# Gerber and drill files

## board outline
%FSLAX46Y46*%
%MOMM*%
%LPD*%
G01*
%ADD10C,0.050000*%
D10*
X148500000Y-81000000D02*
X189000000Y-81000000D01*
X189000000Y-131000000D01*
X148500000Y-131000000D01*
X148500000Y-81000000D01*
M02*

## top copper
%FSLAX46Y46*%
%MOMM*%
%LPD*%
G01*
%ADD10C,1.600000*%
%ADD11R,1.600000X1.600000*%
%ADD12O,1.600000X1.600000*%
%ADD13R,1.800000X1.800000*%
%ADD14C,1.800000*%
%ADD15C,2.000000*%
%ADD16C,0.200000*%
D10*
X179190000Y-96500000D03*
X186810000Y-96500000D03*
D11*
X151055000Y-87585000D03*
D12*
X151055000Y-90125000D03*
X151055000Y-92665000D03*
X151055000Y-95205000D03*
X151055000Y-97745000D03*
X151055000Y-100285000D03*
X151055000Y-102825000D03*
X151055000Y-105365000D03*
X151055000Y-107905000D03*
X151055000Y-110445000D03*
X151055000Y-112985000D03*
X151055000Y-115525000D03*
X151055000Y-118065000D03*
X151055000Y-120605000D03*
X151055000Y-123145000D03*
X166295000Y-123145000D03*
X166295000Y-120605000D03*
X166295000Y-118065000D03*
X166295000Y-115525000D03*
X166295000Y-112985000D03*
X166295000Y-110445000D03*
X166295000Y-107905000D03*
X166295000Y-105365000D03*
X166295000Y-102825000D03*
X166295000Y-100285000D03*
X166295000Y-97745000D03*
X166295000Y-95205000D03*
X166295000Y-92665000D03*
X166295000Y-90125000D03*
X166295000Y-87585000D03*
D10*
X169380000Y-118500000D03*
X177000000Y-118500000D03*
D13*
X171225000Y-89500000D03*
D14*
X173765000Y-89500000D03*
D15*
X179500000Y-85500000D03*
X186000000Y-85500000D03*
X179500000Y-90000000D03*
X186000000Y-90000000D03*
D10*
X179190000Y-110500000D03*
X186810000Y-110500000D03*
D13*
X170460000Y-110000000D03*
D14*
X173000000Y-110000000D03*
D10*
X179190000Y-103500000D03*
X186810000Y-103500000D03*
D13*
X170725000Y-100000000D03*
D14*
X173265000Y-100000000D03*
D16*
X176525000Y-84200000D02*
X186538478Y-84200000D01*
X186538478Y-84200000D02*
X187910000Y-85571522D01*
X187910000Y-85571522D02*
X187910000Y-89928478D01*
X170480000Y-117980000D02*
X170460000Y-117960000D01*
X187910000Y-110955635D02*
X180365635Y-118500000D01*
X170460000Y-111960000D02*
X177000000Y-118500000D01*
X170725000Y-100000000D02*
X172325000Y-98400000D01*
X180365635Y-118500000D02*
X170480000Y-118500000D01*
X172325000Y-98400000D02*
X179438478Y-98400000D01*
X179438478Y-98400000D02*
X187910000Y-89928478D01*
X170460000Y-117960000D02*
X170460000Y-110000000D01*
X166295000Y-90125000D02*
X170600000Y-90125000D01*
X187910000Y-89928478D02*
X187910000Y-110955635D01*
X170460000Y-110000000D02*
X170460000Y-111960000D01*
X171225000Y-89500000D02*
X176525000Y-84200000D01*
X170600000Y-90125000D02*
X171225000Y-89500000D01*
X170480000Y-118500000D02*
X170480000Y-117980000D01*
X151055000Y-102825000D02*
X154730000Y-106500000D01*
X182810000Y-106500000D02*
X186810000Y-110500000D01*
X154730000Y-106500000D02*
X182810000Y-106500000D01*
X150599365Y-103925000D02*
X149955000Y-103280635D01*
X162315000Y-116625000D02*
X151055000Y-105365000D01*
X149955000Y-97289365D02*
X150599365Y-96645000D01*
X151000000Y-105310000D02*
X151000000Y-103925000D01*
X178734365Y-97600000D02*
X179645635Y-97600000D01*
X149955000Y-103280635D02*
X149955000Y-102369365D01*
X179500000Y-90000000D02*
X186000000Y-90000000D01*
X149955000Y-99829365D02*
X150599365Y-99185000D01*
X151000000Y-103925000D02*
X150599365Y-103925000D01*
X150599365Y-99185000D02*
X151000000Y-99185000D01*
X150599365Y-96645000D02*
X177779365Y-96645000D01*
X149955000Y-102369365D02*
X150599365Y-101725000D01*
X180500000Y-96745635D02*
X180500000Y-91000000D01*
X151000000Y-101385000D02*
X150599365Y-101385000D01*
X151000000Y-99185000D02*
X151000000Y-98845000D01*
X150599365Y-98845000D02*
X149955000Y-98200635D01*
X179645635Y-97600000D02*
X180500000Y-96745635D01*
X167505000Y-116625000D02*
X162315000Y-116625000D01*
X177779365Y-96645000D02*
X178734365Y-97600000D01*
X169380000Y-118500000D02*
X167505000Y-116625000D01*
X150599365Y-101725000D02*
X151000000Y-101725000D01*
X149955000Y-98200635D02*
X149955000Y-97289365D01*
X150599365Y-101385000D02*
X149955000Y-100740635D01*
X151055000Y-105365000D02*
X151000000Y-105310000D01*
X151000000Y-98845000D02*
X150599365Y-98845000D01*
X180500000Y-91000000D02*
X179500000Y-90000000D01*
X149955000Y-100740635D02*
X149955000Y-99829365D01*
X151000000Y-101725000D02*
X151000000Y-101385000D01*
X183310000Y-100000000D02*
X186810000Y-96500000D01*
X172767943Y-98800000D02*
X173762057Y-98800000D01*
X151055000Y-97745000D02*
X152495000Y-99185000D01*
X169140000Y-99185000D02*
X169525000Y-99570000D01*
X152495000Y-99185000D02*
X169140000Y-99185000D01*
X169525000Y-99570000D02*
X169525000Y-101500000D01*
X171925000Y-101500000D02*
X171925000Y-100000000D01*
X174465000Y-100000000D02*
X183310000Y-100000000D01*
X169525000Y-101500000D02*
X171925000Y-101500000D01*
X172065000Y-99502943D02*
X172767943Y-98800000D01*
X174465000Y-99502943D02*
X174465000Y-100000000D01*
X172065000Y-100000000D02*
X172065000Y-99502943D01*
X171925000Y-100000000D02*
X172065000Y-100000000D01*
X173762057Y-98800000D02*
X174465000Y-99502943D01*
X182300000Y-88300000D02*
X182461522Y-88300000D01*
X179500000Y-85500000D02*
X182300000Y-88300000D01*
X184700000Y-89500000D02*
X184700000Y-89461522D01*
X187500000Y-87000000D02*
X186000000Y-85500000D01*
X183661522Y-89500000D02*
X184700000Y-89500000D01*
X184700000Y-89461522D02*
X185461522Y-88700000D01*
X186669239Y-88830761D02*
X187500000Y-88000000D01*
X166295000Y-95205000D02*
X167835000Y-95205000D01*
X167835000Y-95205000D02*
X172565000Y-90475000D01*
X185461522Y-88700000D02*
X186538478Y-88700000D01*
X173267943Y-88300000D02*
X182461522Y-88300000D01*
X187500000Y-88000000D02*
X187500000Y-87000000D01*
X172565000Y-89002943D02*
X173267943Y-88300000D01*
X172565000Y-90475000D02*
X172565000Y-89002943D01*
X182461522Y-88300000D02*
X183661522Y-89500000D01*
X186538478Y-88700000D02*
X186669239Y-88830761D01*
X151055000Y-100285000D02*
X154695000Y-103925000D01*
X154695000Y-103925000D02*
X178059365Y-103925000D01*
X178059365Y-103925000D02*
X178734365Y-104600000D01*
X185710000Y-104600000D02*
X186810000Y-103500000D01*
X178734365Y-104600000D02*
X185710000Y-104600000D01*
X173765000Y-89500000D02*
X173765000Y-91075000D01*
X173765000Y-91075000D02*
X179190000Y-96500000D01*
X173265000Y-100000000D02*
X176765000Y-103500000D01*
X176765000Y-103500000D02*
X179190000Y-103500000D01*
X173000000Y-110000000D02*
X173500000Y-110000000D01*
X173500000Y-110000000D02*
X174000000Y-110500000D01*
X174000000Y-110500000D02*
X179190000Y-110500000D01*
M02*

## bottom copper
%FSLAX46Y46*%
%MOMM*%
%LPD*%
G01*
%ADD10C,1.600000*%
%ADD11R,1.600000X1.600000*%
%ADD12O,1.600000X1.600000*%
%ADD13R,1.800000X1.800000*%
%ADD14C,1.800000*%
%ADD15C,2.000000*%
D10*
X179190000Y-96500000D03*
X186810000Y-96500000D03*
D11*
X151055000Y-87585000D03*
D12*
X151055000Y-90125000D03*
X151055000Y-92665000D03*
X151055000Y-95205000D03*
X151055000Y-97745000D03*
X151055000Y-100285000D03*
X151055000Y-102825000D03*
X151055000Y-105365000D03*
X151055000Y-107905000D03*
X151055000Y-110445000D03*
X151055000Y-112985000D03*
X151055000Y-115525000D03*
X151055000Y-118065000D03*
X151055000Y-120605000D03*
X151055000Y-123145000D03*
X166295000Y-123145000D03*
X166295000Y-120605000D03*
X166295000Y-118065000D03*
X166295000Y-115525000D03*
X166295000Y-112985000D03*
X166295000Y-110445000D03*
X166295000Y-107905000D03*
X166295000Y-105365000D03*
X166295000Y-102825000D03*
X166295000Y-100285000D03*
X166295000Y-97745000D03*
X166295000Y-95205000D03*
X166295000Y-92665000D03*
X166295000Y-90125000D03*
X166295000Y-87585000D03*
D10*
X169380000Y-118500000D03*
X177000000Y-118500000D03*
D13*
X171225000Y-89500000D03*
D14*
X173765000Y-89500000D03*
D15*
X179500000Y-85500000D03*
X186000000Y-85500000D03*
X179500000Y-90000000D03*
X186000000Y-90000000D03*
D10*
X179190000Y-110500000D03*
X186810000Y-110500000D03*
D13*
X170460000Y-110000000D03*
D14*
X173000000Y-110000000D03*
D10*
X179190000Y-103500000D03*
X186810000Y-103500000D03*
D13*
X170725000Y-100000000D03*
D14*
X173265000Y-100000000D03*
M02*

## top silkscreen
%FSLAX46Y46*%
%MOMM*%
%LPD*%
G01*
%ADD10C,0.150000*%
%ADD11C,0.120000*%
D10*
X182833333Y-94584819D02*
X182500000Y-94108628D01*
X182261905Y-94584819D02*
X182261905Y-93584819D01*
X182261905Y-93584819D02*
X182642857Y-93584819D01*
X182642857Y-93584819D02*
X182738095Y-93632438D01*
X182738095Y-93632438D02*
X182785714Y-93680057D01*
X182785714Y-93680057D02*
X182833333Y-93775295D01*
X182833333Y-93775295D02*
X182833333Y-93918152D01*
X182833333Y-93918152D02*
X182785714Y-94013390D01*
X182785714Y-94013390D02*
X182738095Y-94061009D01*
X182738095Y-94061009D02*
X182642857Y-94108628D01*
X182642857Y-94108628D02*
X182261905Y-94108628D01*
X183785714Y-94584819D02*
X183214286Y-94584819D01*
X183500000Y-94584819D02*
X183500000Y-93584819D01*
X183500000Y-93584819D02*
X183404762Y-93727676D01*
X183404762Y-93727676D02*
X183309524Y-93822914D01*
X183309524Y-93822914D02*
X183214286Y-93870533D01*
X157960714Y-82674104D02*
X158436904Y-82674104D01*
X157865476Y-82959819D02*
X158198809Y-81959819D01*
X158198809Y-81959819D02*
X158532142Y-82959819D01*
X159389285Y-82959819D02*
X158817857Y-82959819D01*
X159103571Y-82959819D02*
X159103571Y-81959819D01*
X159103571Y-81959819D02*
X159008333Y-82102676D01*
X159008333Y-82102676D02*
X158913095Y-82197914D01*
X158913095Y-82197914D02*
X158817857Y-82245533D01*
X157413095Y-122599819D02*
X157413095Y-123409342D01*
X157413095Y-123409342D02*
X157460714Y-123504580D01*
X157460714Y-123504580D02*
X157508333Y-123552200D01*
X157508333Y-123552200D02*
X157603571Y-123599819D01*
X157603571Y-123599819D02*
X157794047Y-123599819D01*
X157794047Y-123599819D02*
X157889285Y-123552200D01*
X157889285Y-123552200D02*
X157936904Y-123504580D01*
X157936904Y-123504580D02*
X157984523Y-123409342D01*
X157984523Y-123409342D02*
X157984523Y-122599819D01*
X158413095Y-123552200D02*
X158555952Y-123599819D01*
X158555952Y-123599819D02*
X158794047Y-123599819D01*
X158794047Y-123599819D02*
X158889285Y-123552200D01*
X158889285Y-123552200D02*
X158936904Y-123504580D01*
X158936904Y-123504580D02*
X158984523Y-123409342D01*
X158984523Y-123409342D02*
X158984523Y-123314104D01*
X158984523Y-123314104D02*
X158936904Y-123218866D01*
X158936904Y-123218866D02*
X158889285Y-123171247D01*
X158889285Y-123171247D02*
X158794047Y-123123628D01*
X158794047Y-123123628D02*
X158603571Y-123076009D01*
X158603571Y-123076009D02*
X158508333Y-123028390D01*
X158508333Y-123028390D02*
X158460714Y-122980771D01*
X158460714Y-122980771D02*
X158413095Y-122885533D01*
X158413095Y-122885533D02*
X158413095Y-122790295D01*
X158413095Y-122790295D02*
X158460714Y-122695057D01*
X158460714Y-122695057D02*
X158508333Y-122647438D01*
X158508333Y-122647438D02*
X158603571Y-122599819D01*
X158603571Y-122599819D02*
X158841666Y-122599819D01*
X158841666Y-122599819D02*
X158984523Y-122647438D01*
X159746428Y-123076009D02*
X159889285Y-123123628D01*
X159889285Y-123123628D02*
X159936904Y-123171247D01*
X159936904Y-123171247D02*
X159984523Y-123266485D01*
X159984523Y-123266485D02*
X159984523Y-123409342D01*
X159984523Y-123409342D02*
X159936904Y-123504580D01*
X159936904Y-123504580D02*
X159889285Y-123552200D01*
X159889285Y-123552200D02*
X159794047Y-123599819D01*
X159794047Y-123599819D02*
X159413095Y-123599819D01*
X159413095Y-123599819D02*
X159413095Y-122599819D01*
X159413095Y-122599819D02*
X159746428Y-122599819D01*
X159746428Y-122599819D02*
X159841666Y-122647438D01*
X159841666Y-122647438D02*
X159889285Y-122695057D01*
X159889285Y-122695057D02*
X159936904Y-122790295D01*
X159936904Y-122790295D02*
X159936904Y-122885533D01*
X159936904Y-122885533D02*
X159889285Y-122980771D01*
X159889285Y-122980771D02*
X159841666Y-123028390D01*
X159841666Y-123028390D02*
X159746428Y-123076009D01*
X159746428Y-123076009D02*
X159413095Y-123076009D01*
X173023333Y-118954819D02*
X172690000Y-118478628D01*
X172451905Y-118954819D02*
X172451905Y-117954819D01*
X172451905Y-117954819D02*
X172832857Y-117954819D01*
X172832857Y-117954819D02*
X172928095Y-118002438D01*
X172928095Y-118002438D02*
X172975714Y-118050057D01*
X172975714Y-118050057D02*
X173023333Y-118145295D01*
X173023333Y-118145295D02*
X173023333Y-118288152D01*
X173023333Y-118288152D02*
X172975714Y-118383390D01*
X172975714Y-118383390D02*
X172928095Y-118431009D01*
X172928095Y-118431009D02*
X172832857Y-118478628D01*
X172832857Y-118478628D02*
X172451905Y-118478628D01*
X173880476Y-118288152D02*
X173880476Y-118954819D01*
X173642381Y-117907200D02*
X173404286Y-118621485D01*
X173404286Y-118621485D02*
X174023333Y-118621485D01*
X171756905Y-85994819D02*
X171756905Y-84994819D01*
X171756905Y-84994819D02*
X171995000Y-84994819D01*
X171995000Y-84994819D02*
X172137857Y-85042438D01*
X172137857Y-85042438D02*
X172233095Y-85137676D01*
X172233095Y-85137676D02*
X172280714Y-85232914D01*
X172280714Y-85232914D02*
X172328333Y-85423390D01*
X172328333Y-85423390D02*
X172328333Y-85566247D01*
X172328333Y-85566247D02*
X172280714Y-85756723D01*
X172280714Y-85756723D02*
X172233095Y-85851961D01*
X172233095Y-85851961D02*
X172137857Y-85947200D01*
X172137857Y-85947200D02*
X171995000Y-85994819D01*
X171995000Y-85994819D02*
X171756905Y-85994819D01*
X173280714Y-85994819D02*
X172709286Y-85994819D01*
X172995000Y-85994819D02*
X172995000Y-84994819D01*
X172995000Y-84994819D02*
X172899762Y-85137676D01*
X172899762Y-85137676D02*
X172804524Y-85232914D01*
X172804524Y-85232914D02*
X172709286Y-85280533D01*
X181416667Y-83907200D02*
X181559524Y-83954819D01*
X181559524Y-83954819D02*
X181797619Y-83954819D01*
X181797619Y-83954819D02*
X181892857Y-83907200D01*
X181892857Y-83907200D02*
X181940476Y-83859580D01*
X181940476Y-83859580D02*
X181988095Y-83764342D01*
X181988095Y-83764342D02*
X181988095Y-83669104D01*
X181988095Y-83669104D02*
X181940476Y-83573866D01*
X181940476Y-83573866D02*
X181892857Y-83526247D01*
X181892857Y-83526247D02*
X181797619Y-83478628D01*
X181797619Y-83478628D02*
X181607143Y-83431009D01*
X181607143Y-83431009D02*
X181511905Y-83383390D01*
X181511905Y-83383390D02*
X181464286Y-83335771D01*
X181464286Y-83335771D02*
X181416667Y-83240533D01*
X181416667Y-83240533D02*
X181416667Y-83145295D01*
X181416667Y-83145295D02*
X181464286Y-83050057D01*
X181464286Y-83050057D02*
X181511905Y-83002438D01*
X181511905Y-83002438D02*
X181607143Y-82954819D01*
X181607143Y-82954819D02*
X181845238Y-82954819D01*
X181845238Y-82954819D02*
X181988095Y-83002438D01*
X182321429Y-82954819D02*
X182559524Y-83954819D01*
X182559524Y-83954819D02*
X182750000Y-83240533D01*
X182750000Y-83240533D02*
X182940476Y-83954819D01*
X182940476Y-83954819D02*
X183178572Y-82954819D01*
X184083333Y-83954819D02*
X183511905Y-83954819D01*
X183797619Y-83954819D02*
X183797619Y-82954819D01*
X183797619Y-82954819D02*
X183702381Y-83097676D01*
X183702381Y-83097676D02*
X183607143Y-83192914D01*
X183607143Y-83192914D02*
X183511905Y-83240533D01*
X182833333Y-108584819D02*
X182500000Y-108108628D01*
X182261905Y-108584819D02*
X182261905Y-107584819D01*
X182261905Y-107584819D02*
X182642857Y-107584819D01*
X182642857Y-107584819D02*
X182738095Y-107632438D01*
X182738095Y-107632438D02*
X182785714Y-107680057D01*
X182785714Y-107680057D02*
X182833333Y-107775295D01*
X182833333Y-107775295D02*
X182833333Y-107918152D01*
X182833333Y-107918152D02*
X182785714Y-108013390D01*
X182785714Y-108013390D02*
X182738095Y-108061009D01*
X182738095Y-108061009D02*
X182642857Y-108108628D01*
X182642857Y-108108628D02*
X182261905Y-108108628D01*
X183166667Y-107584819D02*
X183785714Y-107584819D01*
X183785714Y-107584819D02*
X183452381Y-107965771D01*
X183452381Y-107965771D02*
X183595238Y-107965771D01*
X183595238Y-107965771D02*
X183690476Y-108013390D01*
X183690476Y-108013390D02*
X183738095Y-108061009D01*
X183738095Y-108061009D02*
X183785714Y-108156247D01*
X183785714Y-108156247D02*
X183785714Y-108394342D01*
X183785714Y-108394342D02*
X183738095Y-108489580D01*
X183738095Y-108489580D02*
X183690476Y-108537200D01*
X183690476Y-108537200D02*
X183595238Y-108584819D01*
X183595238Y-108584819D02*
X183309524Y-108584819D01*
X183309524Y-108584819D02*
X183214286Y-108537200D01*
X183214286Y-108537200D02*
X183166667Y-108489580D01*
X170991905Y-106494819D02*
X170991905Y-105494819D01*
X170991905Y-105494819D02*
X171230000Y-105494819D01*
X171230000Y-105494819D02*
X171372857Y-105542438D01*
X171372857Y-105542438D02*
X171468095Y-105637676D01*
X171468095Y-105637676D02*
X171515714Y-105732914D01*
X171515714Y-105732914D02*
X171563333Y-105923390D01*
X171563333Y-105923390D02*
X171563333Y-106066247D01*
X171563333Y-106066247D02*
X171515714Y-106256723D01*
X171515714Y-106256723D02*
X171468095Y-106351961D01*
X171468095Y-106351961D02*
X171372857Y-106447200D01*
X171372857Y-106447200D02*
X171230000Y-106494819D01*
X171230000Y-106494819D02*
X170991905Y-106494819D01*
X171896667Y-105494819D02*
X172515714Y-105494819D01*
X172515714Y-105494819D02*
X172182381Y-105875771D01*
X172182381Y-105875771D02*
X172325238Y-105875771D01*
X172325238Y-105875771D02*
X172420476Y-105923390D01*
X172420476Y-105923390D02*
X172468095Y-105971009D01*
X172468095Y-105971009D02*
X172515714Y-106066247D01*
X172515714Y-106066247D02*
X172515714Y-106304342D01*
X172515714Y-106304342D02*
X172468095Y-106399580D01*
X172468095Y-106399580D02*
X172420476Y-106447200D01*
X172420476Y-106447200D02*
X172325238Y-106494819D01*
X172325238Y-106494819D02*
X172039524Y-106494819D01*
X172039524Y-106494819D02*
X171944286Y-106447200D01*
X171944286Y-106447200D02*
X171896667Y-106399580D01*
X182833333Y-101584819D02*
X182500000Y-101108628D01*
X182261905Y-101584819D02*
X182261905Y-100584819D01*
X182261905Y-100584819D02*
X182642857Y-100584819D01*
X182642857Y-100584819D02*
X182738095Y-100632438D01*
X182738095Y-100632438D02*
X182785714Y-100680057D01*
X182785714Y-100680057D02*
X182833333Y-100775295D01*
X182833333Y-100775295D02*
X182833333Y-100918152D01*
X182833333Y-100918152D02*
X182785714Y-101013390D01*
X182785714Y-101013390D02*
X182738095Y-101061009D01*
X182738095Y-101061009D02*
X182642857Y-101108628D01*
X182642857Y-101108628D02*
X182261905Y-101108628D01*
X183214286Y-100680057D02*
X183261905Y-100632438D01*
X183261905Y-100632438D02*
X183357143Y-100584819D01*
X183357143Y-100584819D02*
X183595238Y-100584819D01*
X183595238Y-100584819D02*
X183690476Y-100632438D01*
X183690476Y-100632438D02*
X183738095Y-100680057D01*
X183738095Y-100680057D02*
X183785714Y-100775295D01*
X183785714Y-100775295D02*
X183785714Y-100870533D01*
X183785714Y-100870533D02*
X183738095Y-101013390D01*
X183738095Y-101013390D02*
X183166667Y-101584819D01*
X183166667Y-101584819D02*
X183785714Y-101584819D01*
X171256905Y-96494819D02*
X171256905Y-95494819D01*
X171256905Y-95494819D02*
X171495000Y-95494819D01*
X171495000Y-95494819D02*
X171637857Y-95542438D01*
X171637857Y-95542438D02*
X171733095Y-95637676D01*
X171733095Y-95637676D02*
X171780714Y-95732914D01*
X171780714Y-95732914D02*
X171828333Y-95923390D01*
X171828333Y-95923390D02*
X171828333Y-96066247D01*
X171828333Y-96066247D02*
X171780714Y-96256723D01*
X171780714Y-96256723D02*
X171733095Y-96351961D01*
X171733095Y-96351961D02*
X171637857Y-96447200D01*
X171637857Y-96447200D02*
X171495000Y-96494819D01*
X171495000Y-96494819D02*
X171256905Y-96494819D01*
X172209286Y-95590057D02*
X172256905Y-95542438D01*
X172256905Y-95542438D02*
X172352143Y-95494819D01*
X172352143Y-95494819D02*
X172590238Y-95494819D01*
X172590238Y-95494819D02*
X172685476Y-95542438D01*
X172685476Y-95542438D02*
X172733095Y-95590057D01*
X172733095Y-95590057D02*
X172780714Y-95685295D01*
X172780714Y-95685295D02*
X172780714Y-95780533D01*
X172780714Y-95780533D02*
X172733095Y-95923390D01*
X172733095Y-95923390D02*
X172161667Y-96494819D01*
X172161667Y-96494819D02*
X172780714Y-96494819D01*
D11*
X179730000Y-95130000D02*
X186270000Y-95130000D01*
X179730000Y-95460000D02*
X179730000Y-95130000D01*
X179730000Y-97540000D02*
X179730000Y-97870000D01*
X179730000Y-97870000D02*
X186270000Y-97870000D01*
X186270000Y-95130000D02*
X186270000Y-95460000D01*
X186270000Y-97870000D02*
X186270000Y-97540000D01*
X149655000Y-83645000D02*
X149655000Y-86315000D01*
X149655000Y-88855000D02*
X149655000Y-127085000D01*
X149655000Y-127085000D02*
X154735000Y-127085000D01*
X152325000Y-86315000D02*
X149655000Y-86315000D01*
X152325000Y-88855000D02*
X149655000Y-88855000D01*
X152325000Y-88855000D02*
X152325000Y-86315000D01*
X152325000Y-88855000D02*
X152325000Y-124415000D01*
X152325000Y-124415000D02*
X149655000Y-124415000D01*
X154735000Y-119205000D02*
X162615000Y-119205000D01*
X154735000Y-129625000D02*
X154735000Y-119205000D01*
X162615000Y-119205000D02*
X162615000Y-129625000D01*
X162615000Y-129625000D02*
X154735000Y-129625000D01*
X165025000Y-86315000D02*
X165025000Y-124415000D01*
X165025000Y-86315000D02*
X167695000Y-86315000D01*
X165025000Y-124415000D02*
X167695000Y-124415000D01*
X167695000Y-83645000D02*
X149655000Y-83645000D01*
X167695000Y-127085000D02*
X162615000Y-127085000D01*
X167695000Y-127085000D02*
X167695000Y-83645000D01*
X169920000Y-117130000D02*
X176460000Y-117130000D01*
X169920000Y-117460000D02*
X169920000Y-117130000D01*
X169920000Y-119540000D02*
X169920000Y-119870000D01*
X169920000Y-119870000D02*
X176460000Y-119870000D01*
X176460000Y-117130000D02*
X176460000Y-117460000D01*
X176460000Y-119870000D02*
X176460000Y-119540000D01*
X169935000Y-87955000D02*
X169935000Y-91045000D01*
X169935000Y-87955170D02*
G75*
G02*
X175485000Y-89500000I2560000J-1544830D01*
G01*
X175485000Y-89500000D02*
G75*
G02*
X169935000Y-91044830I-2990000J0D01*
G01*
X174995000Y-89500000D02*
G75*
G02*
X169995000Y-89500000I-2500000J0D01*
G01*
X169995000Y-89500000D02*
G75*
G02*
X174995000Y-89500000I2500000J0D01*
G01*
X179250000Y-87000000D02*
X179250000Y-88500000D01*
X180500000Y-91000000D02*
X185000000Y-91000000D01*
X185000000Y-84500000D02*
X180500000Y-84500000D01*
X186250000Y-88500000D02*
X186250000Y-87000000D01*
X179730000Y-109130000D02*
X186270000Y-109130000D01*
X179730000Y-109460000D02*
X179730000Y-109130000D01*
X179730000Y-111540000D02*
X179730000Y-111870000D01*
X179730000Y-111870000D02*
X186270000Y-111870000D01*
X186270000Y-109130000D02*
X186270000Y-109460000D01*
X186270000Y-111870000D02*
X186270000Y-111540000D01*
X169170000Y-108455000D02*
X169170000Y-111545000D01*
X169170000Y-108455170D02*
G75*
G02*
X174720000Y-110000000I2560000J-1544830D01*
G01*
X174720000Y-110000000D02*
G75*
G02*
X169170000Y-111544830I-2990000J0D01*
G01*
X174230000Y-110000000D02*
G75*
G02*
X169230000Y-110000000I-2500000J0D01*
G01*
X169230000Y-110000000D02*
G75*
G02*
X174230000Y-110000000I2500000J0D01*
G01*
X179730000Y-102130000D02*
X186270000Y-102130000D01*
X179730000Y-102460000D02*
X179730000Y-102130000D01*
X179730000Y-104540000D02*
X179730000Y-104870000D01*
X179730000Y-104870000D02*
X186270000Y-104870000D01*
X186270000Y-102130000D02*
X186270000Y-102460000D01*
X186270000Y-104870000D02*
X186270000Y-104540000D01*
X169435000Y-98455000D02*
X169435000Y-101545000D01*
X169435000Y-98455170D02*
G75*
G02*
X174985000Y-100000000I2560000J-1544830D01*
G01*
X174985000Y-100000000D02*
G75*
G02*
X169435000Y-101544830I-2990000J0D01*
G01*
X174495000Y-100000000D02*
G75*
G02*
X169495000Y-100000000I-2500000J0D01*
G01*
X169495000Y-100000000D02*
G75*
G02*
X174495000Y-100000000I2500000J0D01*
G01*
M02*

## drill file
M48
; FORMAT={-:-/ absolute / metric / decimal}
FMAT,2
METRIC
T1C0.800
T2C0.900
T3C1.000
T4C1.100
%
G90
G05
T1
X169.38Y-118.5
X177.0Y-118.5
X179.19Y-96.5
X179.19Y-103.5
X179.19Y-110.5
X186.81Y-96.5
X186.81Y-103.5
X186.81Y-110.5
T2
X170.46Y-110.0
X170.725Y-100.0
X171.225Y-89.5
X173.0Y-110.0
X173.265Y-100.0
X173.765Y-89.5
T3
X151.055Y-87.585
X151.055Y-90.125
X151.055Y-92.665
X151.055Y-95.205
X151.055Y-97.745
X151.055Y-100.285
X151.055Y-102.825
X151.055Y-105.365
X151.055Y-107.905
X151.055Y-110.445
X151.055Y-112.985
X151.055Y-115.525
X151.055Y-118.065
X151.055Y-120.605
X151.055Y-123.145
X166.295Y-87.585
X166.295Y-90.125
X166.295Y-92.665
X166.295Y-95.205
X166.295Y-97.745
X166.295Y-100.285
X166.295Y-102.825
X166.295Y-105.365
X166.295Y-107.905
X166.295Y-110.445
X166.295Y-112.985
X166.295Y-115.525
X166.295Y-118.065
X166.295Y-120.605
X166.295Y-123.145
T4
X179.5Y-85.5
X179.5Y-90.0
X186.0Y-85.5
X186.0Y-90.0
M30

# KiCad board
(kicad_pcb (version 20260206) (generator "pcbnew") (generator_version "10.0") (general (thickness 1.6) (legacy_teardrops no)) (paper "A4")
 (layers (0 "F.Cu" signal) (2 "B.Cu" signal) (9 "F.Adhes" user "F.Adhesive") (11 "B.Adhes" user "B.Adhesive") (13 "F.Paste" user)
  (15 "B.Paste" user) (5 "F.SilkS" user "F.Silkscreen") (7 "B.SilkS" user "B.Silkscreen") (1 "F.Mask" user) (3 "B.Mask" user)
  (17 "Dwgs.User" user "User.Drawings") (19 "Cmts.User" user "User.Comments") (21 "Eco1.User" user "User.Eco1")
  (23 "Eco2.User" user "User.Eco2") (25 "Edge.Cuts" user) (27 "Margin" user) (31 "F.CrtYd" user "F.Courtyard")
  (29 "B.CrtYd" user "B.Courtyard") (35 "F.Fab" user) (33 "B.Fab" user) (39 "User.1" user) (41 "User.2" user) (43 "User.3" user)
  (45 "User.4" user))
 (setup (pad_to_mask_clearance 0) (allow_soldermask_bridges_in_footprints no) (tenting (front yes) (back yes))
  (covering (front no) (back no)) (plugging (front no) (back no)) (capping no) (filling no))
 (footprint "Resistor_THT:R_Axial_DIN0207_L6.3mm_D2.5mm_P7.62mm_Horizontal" (layer "F.Cu") (at 179.19 96.5)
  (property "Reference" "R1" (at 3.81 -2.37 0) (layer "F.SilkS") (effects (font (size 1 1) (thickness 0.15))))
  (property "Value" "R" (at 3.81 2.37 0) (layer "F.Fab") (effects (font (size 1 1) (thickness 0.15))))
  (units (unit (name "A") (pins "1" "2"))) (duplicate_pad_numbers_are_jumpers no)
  (fp_line (start 0.54 -1.37) (end 7.08 -1.37) (stroke (width 0.12) (type solid)) (layer "F.SilkS"))
  (fp_line (start 0.54 -1.04) (end 0.54 -1.37) (stroke (width 0.12) (type solid)) (layer "F.SilkS"))
  (fp_line (start 0.54 1.04) (end 0.54 1.37) (stroke (width 0.12) (type solid)) (layer "F.SilkS"))
  (fp_line (start 0.54 1.37) (end 7.08 1.37) (stroke (width 0.12) (type solid)) (layer "F.SilkS"))
  (fp_line (start 7.08 -1.37) (end 7.08 -1.04) (stroke (width 0.12) (type solid)) (layer "F.SilkS"))
  (fp_line (start 7.08 1.37) (end 7.08 1.04) (stroke (width 0.12) (type solid)) (layer "F.SilkS"))
  (pad "1" thru_hole circle (at 0 0) (size 1.6 1.6) (drill 0.8) (layers "*.Cu" "*.Mask") (remove_unused_layers no) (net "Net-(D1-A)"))
  (pad "2" thru_hole circle (at 7.62 0) (size 1.6 1.6) (drill 0.8) (layers "*.Cu" "*.Mask") (remove_unused_layers no) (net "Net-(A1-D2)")))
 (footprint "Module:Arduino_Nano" (layer "F.Cu") (at 151.055 87.585)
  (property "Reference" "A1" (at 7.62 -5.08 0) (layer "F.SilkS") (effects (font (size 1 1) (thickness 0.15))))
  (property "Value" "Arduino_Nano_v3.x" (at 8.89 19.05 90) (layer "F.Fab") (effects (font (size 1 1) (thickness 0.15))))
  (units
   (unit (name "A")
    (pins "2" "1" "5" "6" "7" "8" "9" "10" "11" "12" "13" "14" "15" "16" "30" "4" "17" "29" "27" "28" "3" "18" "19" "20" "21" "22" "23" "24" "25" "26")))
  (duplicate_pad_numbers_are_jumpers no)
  (fp_line (start -1.4 -3.94) (end -1.4 -1.27) (stroke (width 0.12) (type solid)) (layer "F.SilkS"))
  (fp_line (start -1.4 1.27) (end -1.4 39.5) (stroke (width 0.12) (type solid)) (layer "F.SilkS"))
  (fp_line (start -1.4 39.5) (end 3.68 39.5) (stroke (width 0.12) (type solid)) (layer "F.SilkS"))
  (fp_line (start 1.27 -1.27) (end -1.4 -1.27) (stroke (width 0.12) (type solid)) (layer "F.SilkS"))
  (fp_line (start 1.27 1.27) (end -1.4 1.27) (stroke (width 0.12) (type solid)) (layer "F.SilkS"))
  (fp_line (start 1.27 1.27) (end 1.27 -1.27) (stroke (width 0.12) (type solid)) (layer "F.SilkS"))
  (fp_line (start 1.27 1.27) (end 1.27 36.83) (stroke (width 0.12) (type solid)) (layer "F.SilkS"))
  (fp_line (start 1.27 36.83) (end -1.4 36.83) (stroke (width 0.12) (type solid)) (layer "F.SilkS"))
  (fp_line (start 3.68 31.62) (end 11.56 31.62) (stroke (width 0.12) (type solid)) (layer "F.SilkS"))
  (fp_line (start 3.68 42.04) (end 3.68 31.62) (stroke (width 0.12) (type solid)) (layer "F.SilkS"))
  (fp_line (start 11.56 31.62) (end 11.56 42.04) (stroke (width 0.12) (type solid)) (layer "F.SilkS"))
  (fp_line (start 11.56 42.04) (end 3.68 42.04) (stroke (width 0.12) (type solid)) (layer "F.SilkS"))
  (fp_line (start 13.97 -1.27) (end 13.97 36.83) (stroke (width 0.12) (type solid)) (layer "F.SilkS"))
  (fp_line (start 13.97 -1.27) (end 16.64 -1.27) (stroke (width 0.12) (type solid)) (layer "F.SilkS"))
  (fp_line (start 13.97 36.83) (end 16.64 36.83) (stroke (width 0.12) (type solid)) (layer "F.SilkS"))
  (fp_line (start 16.64 -3.94) (end -1.4 -3.94) (stroke (width 0.12) (type solid)) (layer "F.SilkS"))
  (fp_line (start 16.64 39.5) (end 11.56 39.5) (stroke (width 0.12) (type solid)) (layer "F.SilkS"))
  (fp_line (start 16.64 39.5) (end 16.64 -3.94) (stroke (width 0.12) (type solid)) (layer "F.SilkS"))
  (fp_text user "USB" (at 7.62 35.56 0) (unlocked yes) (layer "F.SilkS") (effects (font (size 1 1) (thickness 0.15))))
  (pad "1" thru_hole rect (at 0 0) (size 1.6 1.6) (drill 1) (layers "*.Cu" "*.Mask") (remove_unused_layers no)
   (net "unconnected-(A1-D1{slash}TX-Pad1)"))
  (pad "2" thru_hole oval (at 0 2.54) (size 1.6 1.6) (drill 1) (layers "*.Cu" "*.Mask") (remove_unused_layers no)
   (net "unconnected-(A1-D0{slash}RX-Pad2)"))
  (pad "3" thru_hole oval (at 0 5.08) (size 1.6 1.6) (drill 1) (layers "*.Cu" "*.Mask") (remove_unused_layers no)
   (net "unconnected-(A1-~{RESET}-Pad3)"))
  (pad "4" thru_hole oval (at 0 7.62) (size 1.6 1.6) (drill 1) (layers "*.Cu" "*.Mask") (remove_unused_layers no)
   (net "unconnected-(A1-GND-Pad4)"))
  (pad "5" thru_hole oval (at 0 10.16) (size 1.6 1.6) (drill 1) (layers "*.Cu" "*.Mask") (remove_unused_layers no) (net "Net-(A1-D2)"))
  (pad "6" thru_hole oval (at 0 12.7) (size 1.6 1.6) (drill 1) (layers "*.Cu" "*.Mask") (remove_unused_layers no) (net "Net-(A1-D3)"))
  (pad "7" thru_hole oval (at 0 15.24) (size 1.6 1.6) (drill 1) (layers "*.Cu" "*.Mask") (remove_unused_layers no) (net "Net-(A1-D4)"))
  (pad "8" thru_hole oval (at 0 17.78) (size 1.6 1.6) (drill 1) (layers "*.Cu" "*.Mask") (remove_unused_layers no) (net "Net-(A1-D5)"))
  (pad "9" thru_hole oval (at 0 20.32) (size 1.6 1.6) (drill 1) (layers "*.Cu" "*.Mask") (remove_unused_layers no)
   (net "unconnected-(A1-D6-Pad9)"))
  (pad "10" thru_hole oval (at 0 22.86) (size 1.6 1.6) (drill 1) (layers "*.Cu" "*.Mask") (remove_unused_layers no)
   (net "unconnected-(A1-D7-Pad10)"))
  (pad "11" thru_hole oval (at 0 25.4) (size 1.6 1.6) (drill 1) (layers "*.Cu" "*.Mask") (remove_unused_layers no)
   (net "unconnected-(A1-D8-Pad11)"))
  (pad "12" thru_hole oval (at 0 27.94) (size 1.6 1.6) (drill 1) (layers "*.Cu" "*.Mask") (remove_unused_layers no)
   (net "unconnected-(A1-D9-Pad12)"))
  (pad "13" thru_hole oval (at 0 30.48) (size 1.6 1.6) (drill 1) (layers "*.Cu" "*.Mask") (remove_unused_layers no)
   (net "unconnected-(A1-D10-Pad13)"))
  (pad "14" thru_hole oval (at 0 33.02) (size 1.6 1.6) (drill 1) (layers "*.Cu" "*.Mask") (remove_unused_layers no)
   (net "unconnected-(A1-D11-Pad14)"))
  (pad "15" thru_hole oval (at 0 35.56) (size 1.6 1.6) (drill 1) (layers "*.Cu" "*.Mask") (remove_unused_layers no)
   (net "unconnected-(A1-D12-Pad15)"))
  (pad "16" thru_hole oval (at 15.24 35.56) (size 1.6 1.6) (drill 1) (layers "*.Cu" "*.Mask") (remove_unused_layers no)
   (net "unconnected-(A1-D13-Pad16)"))
  (pad "17" thru_hole oval (at 15.24 33.02) (size 1.6 1.6) (drill 1) (layers "*.Cu" "*.Mask") (remove_unused_layers no)
   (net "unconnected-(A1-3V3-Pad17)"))
  (pad "18" thru_hole oval (at 15.24 30.48) (size 1.6 1.6) (drill 1) (layers "*.Cu" "*.Mask") (remove_unused_layers no)
   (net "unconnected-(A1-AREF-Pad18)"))
  (pad "19" thru_hole oval (at 15.24 27.94) (size 1.6 1.6) (drill 1) (layers "*.Cu" "*.Mask") (remove_unused_layers no)
   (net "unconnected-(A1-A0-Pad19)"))
  (pad "20" thru_hole oval (at 15.24 25.4) (size 1.6 1.6) (drill 1) (layers "*.Cu" "*.Mask") (remove_unused_layers no)
   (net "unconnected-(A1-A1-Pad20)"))
  (pad "21" thru_hole oval (at 15.24 22.86) (size 1.6 1.6) (drill 1) (layers "*.Cu" "*.Mask") (remove_unused_layers no)
   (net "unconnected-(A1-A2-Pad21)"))
  (pad "22" thru_hole oval (at 15.24 20.32) (size 1.6 1.6) (drill 1) (layers "*.Cu" "*.Mask") (remove_unused_layers no)
   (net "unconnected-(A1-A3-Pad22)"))
  (pad "23" thru_hole oval (at 15.24 17.78) (size 1.6 1.6) (drill 1) (layers "*.Cu" "*.Mask") (remove_unused_layers no)
   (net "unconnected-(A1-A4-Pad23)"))
  (pad "24" thru_hole oval (at 15.24 15.24) (size 1.6 1.6) (drill 1) (layers "*.Cu" "*.Mask") (remove_unused_layers no)
   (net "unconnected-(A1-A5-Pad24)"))
  (pad "25" thru_hole oval (at 15.24 12.7) (size 1.6 1.6) (drill 1) (layers "*.Cu" "*.Mask") (remove_unused_layers no)
   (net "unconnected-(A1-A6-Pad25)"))
  (pad "26" thru_hole oval (at 15.24 10.16) (size 1.6 1.6) (drill 1) (layers "*.Cu" "*.Mask") (remove_unused_layers no)
   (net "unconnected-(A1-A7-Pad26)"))
  (pad "27" thru_hole oval (at 15.24 7.62) (size 1.6 1.6) (drill 1) (layers "*.Cu" "*.Mask") (remove_unused_layers no) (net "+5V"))
  (pad "28" thru_hole oval (at 15.24 5.08) (size 1.6 1.6) (drill 1) (layers "*.Cu" "*.Mask") (remove_unused_layers no)
   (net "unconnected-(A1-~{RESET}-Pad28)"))
  (pad "29" thru_hole oval (at 15.24 2.54) (size 1.6 1.6) (drill 1) (layers "*.Cu" "*.Mask") (remove_unused_layers no) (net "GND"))
  (pad "30" thru_hole oval (at 15.24 0) (size 1.6 1.6) (drill 1) (layers "*.Cu" "*.Mask") (remove_unused_layers no)
   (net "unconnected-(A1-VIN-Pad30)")))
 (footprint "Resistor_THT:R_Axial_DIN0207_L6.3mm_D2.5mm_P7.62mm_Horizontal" (layer "F.Cu") (at 169.38 118.5)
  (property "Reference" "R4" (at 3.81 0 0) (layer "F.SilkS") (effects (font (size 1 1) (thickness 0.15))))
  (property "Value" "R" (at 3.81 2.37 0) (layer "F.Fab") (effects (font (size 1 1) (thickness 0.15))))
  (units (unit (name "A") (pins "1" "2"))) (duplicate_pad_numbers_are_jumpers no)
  (fp_line (start 0.54 -1.37) (end 7.08 -1.37) (stroke (width 0.12) (type solid)) (layer "F.SilkS"))
  (fp_line (start 0.54 -1.04) (end 0.54 -1.37) (stroke (width 0.12) (type solid)) (layer "F.SilkS"))
  (fp_line (start 0.54 1.04) (end 0.54 1.37) (stroke (width 0.12) (type solid)) (layer "F.SilkS"))
  (fp_line (start 0.54 1.37) (end 7.08 1.37) (stroke (width 0.12) (type solid)) (layer "F.SilkS"))
  (fp_line (start 7.08 -1.37) (end 7.08 -1.04) (stroke (width 0.12) (type solid)) (layer "F.SilkS"))
  (fp_line (start 7.08 1.37) (end 7.08 1.04) (stroke (width 0.12) (type solid)) (layer "F.SilkS"))
  (pad "1" thru_hole circle (at 0 0) (size 1.6 1.6) (drill 0.8) (layers "*.Cu" "*.Mask") (remove_unused_layers no) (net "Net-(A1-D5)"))
  (pad "2" thru_hole circle (at 7.62 0) (size 1.6 1.6) (drill 0.8) (layers "*.Cu" "*.Mask") (remove_unused_layers no) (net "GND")))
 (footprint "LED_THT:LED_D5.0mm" (layer "F.Cu") (at 171.225 89.5)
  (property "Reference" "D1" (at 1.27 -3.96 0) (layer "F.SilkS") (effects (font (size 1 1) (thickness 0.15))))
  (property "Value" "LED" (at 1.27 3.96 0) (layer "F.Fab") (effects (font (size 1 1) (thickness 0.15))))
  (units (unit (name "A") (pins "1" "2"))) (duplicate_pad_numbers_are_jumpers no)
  (fp_line (start -1.29 -1.545) (end -1.29 1.545) (stroke (width 0.12) (type solid)) (layer "F.SilkS"))
  (fp_arc (start -1.29 -1.54483) (mid 2.071779 -2.880495) (end 4.26 0) (stroke (width 0.12) (type solid)) (layer "F.SilkS"))
  (fp_arc (start 4.26 0) (mid 2.071779 2.880495) (end -1.29 1.54483) (stroke (width 0.12) (type solid)) (layer "F.SilkS"))
  (fp_circle (center 1.27 0) (end 3.77 0) (stroke (width 0.12) (type solid)) (fill no) (layer "F.SilkS"))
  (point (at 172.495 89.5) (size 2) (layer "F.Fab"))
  (pad "1" thru_hole rect (at 0 0) (size 1.8 1.8) (drill 0.9) (layers "*.Cu" "*.Mask") (remove_unused_layers no) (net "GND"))
  (pad "2" thru_hole circle (at 2.54 0) (size 1.8 1.8) (drill 0.9) (layers "*.Cu" "*.Mask") (remove_unused_layers no) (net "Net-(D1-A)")))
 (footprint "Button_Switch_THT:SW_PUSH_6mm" (layer "F.Cu") (at 179.5 85.5)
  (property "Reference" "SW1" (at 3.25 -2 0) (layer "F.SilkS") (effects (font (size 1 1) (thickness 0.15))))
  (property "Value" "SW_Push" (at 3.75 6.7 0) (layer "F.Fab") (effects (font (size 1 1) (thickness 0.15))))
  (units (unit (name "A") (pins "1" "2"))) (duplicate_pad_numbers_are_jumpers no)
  (fp_line (start -0.25 1.5) (end -0.25 3) (stroke (width 0.12) (type solid)) (layer "F.SilkS"))
  (fp_line (start 1 5.5) (end 5.5 5.5) (stroke (width 0.12) (type solid)) (layer "F.SilkS"))
  (fp_line (start 5.5 -1) (end 1 -1) (stroke (width 0.12) (type solid)) (layer "F.SilkS"))
  (fp_line (start 6.75 3) (end 6.75 1.5) (stroke (width 0.12) (type solid)) (layer "F.SilkS"))
  (pad "1" thru_hole circle (at 0 0 90) (size 2 2) (drill 1.1) (layers "*.Cu" "*.Mask") (remove_unused_layers no) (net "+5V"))
  (pad "1" thru_hole circle (at 6.5 0 90) (size 2 2) (drill 1.1) (layers "*.Cu" "*.Mask") (remove_unused_layers no) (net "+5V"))
  (pad "2" thru_hole circle (at 0 4.5 90) (size 2 2) (drill 1.1) (layers "*.Cu" "*.Mask") (remove_unused_layers no) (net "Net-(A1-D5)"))
  (pad "2" thru_hole circle (at 6.5 4.5 90) (size 2 2) (drill 1.1) (layers "*.Cu" "*.Mask") (remove_unused_layers no) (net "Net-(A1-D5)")))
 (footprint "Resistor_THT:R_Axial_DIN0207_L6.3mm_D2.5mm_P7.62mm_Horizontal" (layer "F.Cu") (at 179.19 110.5)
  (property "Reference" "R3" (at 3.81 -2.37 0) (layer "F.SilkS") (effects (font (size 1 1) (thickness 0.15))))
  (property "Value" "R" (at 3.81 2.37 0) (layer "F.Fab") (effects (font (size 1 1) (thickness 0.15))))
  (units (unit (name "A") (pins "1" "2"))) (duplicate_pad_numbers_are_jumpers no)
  (fp_line (start 0.54 -1.37) (end 7.08 -1.37) (stroke (width 0.12) (type solid)) (layer "F.SilkS"))
  (fp_line (start 0.54 -1.04) (end 0.54 -1.37) (stroke (width 0.12) (type solid)) (layer "F.SilkS"))
  (fp_line (start 0.54 1.04) (end 0.54 1.37) (stroke (width 0.12) (type solid)) (layer "F.SilkS"))
  (fp_line (start 0.54 1.37) (end 7.08 1.37) (stroke (width 0.12) (type solid)) (layer "F.SilkS"))
  (fp_line (start 7.08 -1.37) (end 7.08 -1.04) (stroke (width 0.12) (type solid)) (layer "F.SilkS"))
  (fp_line (start 7.08 1.37) (end 7.08 1.04) (stroke (width 0.12) (type solid)) (layer "F.SilkS"))
  (pad "1" thru_hole circle (at 0 0) (size 1.6 1.6) (drill 0.8) (layers "*.Cu" "*.Mask") (remove_unused_layers no) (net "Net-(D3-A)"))
  (pad "2" thru_hole circle (at 7.62 0) (size 1.6 1.6) (drill 0.8) (layers "*.Cu" "*.Mask") (remove_unused_layers no) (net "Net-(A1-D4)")))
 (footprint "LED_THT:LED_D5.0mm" (layer "F.Cu") (at 170.46 110)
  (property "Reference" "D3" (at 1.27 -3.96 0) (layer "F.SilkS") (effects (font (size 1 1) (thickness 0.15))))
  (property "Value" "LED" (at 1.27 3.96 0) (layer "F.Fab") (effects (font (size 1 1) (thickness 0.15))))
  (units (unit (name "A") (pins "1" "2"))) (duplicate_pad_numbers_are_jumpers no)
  (fp_line (start -1.29 -1.545) (end -1.29 1.545) (stroke (width 0.12) (type solid)) (layer "F.SilkS"))
  (fp_arc (start -1.29 -1.54483) (mid 2.071779 -2.880495) (end 4.26 0) (stroke (width 0.12) (type solid)) (layer "F.SilkS"))
  (fp_arc (start 4.26 0) (mid 2.071779 2.880495) (end -1.29 1.54483) (stroke (width 0.12) (type solid)) (layer "F.SilkS"))
  (fp_circle (center 1.27 0) (end 3.77 0) (stroke (width 0.12) (type solid)) (fill no) (layer "F.SilkS"))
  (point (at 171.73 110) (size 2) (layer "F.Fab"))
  (pad "1" thru_hole rect (at 0 0) (size 1.8 1.8) (drill 0.9) (layers "*.Cu" "*.Mask") (remove_unused_layers no) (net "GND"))
  (pad "2" thru_hole circle (at 2.54 0) (size 1.8 1.8) (drill 0.9) (layers "*.Cu" "*.Mask") (remove_unused_layers no) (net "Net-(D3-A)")))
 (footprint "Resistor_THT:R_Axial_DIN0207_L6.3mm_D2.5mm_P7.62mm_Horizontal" (layer "F.Cu") (at 179.19 103.5)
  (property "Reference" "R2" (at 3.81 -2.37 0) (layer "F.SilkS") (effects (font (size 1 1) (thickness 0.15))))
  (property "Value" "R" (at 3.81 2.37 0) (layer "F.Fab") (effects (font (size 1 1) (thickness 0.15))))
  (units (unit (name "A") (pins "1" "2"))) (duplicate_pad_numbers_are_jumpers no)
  (fp_line (start 0.54 -1.37) (end 7.08 -1.37) (stroke (width 0.12) (type solid)) (layer "F.SilkS"))
  (fp_line (start 0.54 -1.04) (end 0.54 -1.37) (stroke (width 0.12) (type solid)) (layer "F.SilkS"))
  (fp_line (start 0.54 1.04) (end 0.54 1.37) (stroke (width 0.12) (type solid)) (layer "F.SilkS"))
  (fp_line (start 0.54 1.37) (end 7.08 1.37) (stroke (width 0.12) (type solid)) (layer "F.SilkS"))
  (fp_line (start 7.08 -1.37) (end 7.08 -1.04) (stroke (width 0.12) (type solid)) (layer "F.SilkS"))
  (fp_line (start 7.08 1.37) (end 7.08 1.04) (stroke (width 0.12) (type solid)) (layer "F.SilkS"))
  (pad "1" thru_hole circle (at 0 0) (size 1.6 1.6) (drill 0.8) (layers "*.Cu" "*.Mask") (remove_unused_layers no) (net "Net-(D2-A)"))
  (pad "2" thru_hole circle (at 7.62 0) (size 1.6 1.6) (drill 0.8) (layers "*.Cu" "*.Mask") (remove_unused_layers no) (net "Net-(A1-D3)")))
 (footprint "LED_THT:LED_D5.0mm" (layer "F.Cu") (at 170.725 100)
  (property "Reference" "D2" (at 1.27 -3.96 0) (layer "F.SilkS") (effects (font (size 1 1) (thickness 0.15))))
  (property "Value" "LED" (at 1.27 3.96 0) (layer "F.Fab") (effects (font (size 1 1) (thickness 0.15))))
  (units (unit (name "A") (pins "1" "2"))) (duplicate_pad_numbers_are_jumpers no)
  (fp_line (start -1.29 -1.545) (end -1.29 1.545) (stroke (width 0.12) (type solid)) (layer "F.SilkS"))
  (fp_arc (start -1.29 -1.54483) (mid 2.071779 -2.880495) (end 4.26 0) (stroke (width 0.12) (type solid)) (layer "F.SilkS"))
  (fp_arc (start 4.26 0) (mid 2.071779 2.880495) (end -1.29 1.54483) (stroke (width 0.12) (type solid)) (layer "F.SilkS"))
  (fp_circle (center 1.27 0) (end 3.77 0) (stroke (width 0.12) (type solid)) (fill no) (layer "F.SilkS"))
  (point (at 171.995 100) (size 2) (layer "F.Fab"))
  (pad "1" thru_hole rect (at 0 0) (size 1.8 1.8) (drill 0.9) (layers "*.Cu" "*.Mask") (remove_unused_layers no) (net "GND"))
  (pad "2" thru_hole circle (at 2.54 0) (size 1.8 1.8) (drill 0.9) (layers "*.Cu" "*.Mask") (remove_unused_layers no) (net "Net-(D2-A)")))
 (gr_rect (start 148.5 81) (end 189 131) (stroke (width 0.05) (type default)) (fill no) (layer "Edge.Cuts"))
 (segment (start 176.525 84.2) (end 186.538478 84.2) (width 0.2) (layer "F.Cu") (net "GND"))
 (segment (start 186.538478 84.2) (end 187.91 85.571522) (width 0.2) (layer "F.Cu") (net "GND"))
 (segment (start 187.91 85.571522) (end 187.91 89.928478) (width 0.2) (layer "F.Cu") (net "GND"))
 (segment (start 170.48 117.98) (end 170.46 117.96) (width 0.2) (layer "F.Cu") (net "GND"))
 (segment (start 187.91 110.955635) (end 180.365635 118.5) (width 0.2) (layer "F.Cu") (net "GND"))
 (segment (start 170.46 111.96) (end 177 118.5) (width 0.2) (layer "F.Cu") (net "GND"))
 (segment (start 170.725 100) (end 172.325 98.4) (width 0.2) (layer "F.Cu") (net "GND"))
 (segment (start 180.365635 118.5) (end 170.48 118.5) (width 0.2) (layer "F.Cu") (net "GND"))
 (segment (start 172.325 98.4) (end 179.438478 98.4) (width 0.2) (layer "F.Cu") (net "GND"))
 (segment (start 179.438478 98.4) (end 187.91 89.928478) (width 0.2) (layer "F.Cu") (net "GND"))
 (segment (start 170.46 117.96) (end 170.46 110) (width 0.2) (layer "F.Cu") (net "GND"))
 (segment (start 166.295 90.125) (end 170.6 90.125) (width 0.2) (layer "F.Cu") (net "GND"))
 (segment (start 187.91 89.928478) (end 187.91 110.955635) (width 0.2) (layer "F.Cu") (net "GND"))
 (segment (start 170.46 110) (end 170.46 111.96) (width 0.2) (layer "F.Cu") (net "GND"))
 (segment (start 171.225 89.5) (end 176.525 84.2) (width 0.2) (layer "F.Cu") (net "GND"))
 (segment (start 170.6 90.125) (end 171.225 89.5) (width 0.2) (layer "F.Cu") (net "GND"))
 (segment (start 170.48 118.5) (end 170.48 117.98) (width 0.2) (layer "F.Cu") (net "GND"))
 (segment (start 151.055 102.825) (end 154.73 106.5) (width 0.2) (layer "F.Cu") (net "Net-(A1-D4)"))
 (segment (start 182.81 106.5) (end 186.81 110.5) (width 0.2) (layer "F.Cu") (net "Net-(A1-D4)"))
 (segment (start 154.73 106.5) (end 182.81 106.5) (width 0.2) (layer "F.Cu") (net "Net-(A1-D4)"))
 (segment (start 150.599365 103.925) (end 149.955 103.280635) (width 0.2) (layer "F.Cu") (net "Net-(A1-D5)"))
 (segment (start 162.315 116.625) (end 151.055 105.365) (width 0.2) (layer "F.Cu") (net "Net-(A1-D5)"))
 (segment (start 149.955 97.289365) (end 150.599365 96.645) (width 0.2) (layer "F.Cu") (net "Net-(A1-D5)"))
 (segment (start 151 105.31) (end 151 103.925) (width 0.2) (layer "F.Cu") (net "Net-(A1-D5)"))
 (segment (start 178.734365 97.6) (end 179.645635 97.6) (width 0.2) (layer "F.Cu") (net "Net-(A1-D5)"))
 (segment (start 149.955 103.280635) (end 149.955 102.369365) (width 0.2) (layer "F.Cu") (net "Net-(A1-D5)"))
 (segment (start 179.5 90) (end 186 90) (width 0.2) (layer "F.Cu") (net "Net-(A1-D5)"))
 (segment (start 149.955 99.829365) (end 150.599365 99.185) (width 0.2) (layer "F.Cu") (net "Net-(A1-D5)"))
 (segment (start 151 103.925) (end 150.599365 103.925) (width 0.2) (layer "F.Cu") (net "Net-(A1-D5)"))
 (segment (start 150.599365 99.185) (end 151 99.185) (width 0.2) (layer "F.Cu") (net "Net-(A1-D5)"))
 (segment (start 150.599365 96.645) (end 177.779365 96.645) (width 0.2) (layer "F.Cu") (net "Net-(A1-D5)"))
 (segment (start 149.955 102.369365) (end 150.599365 101.725) (width 0.2) (layer "F.Cu") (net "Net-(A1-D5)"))
 (segment (start 180.5 96.745635) (end 180.5 91) (width 0.2) (layer "F.Cu") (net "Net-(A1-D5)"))
 (segment (start 151 101.385) (end 150.599365 101.385) (width 0.2) (layer "F.Cu") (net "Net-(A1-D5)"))
 (segment (start 151 99.185) (end 151 98.845) (width 0.2) (layer "F.Cu") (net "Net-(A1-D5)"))
 (segment (start 150.599365 98.845) (end 149.955 98.200635) (width 0.2) (layer "F.Cu") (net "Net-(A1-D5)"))
 (segment (start 179.645635 97.6) (end 180.5 96.745635) (width 0.2) (layer "F.Cu") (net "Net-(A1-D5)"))
 (segment (start 167.505 116.625) (end 162.315 116.625) (width 0.2) (layer "F.Cu") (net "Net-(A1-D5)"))
 (segment (start 177.779365 96.645) (end 178.734365 97.6) (width 0.2) (layer "F.Cu") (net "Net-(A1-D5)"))
 (segment (start 169.38 118.5) (end 167.505 116.625) (width 0.2) (layer "F.Cu") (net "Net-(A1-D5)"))
 (segment (start 150.599365 101.725) (end 151 101.725) (width 0.2) (layer "F.Cu") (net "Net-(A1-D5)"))
 (segment (start 149.955 98.200635) (end 149.955 97.289365) (width 0.2) (layer "F.Cu") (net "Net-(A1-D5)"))
 (segment (start 150.599365 101.385) (end 149.955 100.740635) (width 0.2) (layer "F.Cu") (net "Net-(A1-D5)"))
 (segment (start 151.055 105.365) (end 151 105.31) (width 0.2) (layer "F.Cu") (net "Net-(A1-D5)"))
 (segment (start 151 98.845) (end 150.599365 98.845) (width 0.2) (layer "F.Cu") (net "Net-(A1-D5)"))
 (segment (start 180.5 91) (end 179.5 90) (width 0.2) (layer "F.Cu") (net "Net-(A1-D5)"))
 (segment (start 149.955 100.740635) (end 149.955 99.829365) (width 0.2) (layer "F.Cu") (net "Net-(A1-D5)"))
 (segment (start 151 101.725) (end 151 101.385) (width 0.2) (layer "F.Cu") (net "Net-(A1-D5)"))
 (segment (start 183.31 100) (end 186.81 96.5) (width 0.2) (layer "F.Cu") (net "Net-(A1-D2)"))
 (segment (start 172.767943 98.8) (end 173.762057 98.8) (width 0.2) (layer "F.Cu") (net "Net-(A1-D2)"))
 (segment (start 151.055 97.745) (end 152.495 99.185) (width 0.2) (layer "F.Cu") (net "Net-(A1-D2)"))
 (segment (start 169.14 99.185) (end 169.525 99.57) (width 0.2) (layer "F.Cu") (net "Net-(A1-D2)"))
 (segment (start 152.495 99.185) (end 169.14 99.185) (width 0.2) (layer "F.Cu") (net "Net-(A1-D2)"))
 (segment (start 169.525 99.57) (end 169.525 101.5) (width 0.2) (layer "F.Cu") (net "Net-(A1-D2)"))
 (segment (start 171.925 101.5) (end 171.925 100) (width 0.2) (layer "F.Cu") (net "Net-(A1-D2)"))
 (segment (start 174.465 100) (end 183.31 100) (width 0.2) (layer "F.Cu") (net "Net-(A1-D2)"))
 (segment (start 169.525 101.5) (end 171.925 101.5) (width 0.2) (layer "F.Cu") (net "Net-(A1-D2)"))
 (segment (start 172.065 99.502943) (end 172.767943 98.8) (width 0.2) (layer "F.Cu") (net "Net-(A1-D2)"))
 (segment (start 174.465 99.502943) (end 174.465 100) (width 0.2) (layer "F.Cu") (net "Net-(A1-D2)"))
 (segment (start 172.065 100) (end 172.065 99.502943) (width 0.2) (layer "F.Cu") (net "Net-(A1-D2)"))
 (segment (start 171.925 100) (end 172.065 100) (width 0.2) (layer "F.Cu") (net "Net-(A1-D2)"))
 (segment (start 173.762057 98.8) (end 174.465 99.502943) (width 0.2) (layer "F.Cu") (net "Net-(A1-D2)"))
 (segment (start 182.3 88.3) (end 182.461522 88.3) (width 0.2) (layer "F.Cu") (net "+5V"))
 (segment (start 179.5 85.5) (end 182.3 88.3) (width 0.2) (layer "F.Cu") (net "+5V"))
 (segment (start 184.7 89.5) (end 184.7 89.461522) (width 0.2) (layer "F.Cu") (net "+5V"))
 (segment (start 187.5 87) (end 186 85.5) (width 0.2) (layer "F.Cu") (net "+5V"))
 (segment (start 183.661522 89.5) (end 184.7 89.5) (width 0.2) (layer "F.Cu") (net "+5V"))
 (segment (start 184.7 89.461522) (end 185.461522 88.7) (width 0.2) (layer "F.Cu") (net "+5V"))
 (segment (start 186.669239 88.830761) (end 187.5 88) (width 0.2) (layer "F.Cu") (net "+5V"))
 (segment (start 166.295 95.205) (end 167.835 95.205) (width 0.2) (layer "F.Cu") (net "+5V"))
 (segment (start 167.835 95.205) (end 172.565 90.475) (width 0.2) (layer "F.Cu") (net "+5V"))
 (segment (start 185.461522 88.7) (end 186.538478 88.7) (width 0.2) (layer "F.Cu") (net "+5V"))
 (segment (start 173.267943 88.3) (end 182.461522 88.3) (width 0.2) (layer "F.Cu") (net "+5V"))
 (segment (start 187.5 88) (end 187.5 87) (width 0.2) (layer "F.Cu") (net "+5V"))
 (segment (start 172.565 89.002943) (end 173.267943 88.3) (width 0.2) (layer "F.Cu") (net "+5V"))
 (segment (start 172.565 90.475) (end 172.565 89.002943) (width 0.2) (layer "F.Cu") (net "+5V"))
 (segment (start 182.461522 88.3) (end 183.661522 89.5) (width 0.2) (layer "F.Cu") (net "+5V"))
 (segment (start 186.538478 88.7) (end 186.669239 88.830761) (width 0.2) (layer "F.Cu") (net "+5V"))
 (segment (start 151.055 100.285) (end 154.695 103.925) (width 0.2) (layer "F.Cu") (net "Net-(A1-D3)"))
 (segment (start 154.695 103.925) (end 178.059365 103.925) (width 0.2) (layer "F.Cu") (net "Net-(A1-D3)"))
 (segment (start 178.059365 103.925) (end 178.734365 104.6) (width 0.2) (layer "F.Cu") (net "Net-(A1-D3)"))
 (segment (start 185.71 104.6) (end 186.81 103.5) (width 0.2) (layer "F.Cu") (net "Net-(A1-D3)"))
 (segment (start 178.734365 104.6) (end 185.71 104.6) (width 0.2) (layer "F.Cu") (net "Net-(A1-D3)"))
 (segment (start 173.765 89.5) (end 173.765 91.075) (width 0.2) (layer "F.Cu") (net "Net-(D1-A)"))
 (segment (start 173.765 91.075) (end 179.19 96.5) (width 0.2) (layer "F.Cu") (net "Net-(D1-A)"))
 (segment (start 173.265 100) (end 176.765 103.5) (width 0.2) (layer "F.Cu") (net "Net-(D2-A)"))
 (segment (start 176.765 103.5) (end 179.19 103.5) (width 0.2) (layer "F.Cu") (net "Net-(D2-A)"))
 (segment (start 173 110) (end 173.5 110) (width 0.2) (layer "F.Cu") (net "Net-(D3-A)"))
 (segment (start 173.5 110) (end 174 110.5) (width 0.2) (layer "F.Cu") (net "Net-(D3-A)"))
 (segment (start 174 110.5) (end 179.19 110.5) (width 0.2) (layer "F.Cu") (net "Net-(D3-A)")))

